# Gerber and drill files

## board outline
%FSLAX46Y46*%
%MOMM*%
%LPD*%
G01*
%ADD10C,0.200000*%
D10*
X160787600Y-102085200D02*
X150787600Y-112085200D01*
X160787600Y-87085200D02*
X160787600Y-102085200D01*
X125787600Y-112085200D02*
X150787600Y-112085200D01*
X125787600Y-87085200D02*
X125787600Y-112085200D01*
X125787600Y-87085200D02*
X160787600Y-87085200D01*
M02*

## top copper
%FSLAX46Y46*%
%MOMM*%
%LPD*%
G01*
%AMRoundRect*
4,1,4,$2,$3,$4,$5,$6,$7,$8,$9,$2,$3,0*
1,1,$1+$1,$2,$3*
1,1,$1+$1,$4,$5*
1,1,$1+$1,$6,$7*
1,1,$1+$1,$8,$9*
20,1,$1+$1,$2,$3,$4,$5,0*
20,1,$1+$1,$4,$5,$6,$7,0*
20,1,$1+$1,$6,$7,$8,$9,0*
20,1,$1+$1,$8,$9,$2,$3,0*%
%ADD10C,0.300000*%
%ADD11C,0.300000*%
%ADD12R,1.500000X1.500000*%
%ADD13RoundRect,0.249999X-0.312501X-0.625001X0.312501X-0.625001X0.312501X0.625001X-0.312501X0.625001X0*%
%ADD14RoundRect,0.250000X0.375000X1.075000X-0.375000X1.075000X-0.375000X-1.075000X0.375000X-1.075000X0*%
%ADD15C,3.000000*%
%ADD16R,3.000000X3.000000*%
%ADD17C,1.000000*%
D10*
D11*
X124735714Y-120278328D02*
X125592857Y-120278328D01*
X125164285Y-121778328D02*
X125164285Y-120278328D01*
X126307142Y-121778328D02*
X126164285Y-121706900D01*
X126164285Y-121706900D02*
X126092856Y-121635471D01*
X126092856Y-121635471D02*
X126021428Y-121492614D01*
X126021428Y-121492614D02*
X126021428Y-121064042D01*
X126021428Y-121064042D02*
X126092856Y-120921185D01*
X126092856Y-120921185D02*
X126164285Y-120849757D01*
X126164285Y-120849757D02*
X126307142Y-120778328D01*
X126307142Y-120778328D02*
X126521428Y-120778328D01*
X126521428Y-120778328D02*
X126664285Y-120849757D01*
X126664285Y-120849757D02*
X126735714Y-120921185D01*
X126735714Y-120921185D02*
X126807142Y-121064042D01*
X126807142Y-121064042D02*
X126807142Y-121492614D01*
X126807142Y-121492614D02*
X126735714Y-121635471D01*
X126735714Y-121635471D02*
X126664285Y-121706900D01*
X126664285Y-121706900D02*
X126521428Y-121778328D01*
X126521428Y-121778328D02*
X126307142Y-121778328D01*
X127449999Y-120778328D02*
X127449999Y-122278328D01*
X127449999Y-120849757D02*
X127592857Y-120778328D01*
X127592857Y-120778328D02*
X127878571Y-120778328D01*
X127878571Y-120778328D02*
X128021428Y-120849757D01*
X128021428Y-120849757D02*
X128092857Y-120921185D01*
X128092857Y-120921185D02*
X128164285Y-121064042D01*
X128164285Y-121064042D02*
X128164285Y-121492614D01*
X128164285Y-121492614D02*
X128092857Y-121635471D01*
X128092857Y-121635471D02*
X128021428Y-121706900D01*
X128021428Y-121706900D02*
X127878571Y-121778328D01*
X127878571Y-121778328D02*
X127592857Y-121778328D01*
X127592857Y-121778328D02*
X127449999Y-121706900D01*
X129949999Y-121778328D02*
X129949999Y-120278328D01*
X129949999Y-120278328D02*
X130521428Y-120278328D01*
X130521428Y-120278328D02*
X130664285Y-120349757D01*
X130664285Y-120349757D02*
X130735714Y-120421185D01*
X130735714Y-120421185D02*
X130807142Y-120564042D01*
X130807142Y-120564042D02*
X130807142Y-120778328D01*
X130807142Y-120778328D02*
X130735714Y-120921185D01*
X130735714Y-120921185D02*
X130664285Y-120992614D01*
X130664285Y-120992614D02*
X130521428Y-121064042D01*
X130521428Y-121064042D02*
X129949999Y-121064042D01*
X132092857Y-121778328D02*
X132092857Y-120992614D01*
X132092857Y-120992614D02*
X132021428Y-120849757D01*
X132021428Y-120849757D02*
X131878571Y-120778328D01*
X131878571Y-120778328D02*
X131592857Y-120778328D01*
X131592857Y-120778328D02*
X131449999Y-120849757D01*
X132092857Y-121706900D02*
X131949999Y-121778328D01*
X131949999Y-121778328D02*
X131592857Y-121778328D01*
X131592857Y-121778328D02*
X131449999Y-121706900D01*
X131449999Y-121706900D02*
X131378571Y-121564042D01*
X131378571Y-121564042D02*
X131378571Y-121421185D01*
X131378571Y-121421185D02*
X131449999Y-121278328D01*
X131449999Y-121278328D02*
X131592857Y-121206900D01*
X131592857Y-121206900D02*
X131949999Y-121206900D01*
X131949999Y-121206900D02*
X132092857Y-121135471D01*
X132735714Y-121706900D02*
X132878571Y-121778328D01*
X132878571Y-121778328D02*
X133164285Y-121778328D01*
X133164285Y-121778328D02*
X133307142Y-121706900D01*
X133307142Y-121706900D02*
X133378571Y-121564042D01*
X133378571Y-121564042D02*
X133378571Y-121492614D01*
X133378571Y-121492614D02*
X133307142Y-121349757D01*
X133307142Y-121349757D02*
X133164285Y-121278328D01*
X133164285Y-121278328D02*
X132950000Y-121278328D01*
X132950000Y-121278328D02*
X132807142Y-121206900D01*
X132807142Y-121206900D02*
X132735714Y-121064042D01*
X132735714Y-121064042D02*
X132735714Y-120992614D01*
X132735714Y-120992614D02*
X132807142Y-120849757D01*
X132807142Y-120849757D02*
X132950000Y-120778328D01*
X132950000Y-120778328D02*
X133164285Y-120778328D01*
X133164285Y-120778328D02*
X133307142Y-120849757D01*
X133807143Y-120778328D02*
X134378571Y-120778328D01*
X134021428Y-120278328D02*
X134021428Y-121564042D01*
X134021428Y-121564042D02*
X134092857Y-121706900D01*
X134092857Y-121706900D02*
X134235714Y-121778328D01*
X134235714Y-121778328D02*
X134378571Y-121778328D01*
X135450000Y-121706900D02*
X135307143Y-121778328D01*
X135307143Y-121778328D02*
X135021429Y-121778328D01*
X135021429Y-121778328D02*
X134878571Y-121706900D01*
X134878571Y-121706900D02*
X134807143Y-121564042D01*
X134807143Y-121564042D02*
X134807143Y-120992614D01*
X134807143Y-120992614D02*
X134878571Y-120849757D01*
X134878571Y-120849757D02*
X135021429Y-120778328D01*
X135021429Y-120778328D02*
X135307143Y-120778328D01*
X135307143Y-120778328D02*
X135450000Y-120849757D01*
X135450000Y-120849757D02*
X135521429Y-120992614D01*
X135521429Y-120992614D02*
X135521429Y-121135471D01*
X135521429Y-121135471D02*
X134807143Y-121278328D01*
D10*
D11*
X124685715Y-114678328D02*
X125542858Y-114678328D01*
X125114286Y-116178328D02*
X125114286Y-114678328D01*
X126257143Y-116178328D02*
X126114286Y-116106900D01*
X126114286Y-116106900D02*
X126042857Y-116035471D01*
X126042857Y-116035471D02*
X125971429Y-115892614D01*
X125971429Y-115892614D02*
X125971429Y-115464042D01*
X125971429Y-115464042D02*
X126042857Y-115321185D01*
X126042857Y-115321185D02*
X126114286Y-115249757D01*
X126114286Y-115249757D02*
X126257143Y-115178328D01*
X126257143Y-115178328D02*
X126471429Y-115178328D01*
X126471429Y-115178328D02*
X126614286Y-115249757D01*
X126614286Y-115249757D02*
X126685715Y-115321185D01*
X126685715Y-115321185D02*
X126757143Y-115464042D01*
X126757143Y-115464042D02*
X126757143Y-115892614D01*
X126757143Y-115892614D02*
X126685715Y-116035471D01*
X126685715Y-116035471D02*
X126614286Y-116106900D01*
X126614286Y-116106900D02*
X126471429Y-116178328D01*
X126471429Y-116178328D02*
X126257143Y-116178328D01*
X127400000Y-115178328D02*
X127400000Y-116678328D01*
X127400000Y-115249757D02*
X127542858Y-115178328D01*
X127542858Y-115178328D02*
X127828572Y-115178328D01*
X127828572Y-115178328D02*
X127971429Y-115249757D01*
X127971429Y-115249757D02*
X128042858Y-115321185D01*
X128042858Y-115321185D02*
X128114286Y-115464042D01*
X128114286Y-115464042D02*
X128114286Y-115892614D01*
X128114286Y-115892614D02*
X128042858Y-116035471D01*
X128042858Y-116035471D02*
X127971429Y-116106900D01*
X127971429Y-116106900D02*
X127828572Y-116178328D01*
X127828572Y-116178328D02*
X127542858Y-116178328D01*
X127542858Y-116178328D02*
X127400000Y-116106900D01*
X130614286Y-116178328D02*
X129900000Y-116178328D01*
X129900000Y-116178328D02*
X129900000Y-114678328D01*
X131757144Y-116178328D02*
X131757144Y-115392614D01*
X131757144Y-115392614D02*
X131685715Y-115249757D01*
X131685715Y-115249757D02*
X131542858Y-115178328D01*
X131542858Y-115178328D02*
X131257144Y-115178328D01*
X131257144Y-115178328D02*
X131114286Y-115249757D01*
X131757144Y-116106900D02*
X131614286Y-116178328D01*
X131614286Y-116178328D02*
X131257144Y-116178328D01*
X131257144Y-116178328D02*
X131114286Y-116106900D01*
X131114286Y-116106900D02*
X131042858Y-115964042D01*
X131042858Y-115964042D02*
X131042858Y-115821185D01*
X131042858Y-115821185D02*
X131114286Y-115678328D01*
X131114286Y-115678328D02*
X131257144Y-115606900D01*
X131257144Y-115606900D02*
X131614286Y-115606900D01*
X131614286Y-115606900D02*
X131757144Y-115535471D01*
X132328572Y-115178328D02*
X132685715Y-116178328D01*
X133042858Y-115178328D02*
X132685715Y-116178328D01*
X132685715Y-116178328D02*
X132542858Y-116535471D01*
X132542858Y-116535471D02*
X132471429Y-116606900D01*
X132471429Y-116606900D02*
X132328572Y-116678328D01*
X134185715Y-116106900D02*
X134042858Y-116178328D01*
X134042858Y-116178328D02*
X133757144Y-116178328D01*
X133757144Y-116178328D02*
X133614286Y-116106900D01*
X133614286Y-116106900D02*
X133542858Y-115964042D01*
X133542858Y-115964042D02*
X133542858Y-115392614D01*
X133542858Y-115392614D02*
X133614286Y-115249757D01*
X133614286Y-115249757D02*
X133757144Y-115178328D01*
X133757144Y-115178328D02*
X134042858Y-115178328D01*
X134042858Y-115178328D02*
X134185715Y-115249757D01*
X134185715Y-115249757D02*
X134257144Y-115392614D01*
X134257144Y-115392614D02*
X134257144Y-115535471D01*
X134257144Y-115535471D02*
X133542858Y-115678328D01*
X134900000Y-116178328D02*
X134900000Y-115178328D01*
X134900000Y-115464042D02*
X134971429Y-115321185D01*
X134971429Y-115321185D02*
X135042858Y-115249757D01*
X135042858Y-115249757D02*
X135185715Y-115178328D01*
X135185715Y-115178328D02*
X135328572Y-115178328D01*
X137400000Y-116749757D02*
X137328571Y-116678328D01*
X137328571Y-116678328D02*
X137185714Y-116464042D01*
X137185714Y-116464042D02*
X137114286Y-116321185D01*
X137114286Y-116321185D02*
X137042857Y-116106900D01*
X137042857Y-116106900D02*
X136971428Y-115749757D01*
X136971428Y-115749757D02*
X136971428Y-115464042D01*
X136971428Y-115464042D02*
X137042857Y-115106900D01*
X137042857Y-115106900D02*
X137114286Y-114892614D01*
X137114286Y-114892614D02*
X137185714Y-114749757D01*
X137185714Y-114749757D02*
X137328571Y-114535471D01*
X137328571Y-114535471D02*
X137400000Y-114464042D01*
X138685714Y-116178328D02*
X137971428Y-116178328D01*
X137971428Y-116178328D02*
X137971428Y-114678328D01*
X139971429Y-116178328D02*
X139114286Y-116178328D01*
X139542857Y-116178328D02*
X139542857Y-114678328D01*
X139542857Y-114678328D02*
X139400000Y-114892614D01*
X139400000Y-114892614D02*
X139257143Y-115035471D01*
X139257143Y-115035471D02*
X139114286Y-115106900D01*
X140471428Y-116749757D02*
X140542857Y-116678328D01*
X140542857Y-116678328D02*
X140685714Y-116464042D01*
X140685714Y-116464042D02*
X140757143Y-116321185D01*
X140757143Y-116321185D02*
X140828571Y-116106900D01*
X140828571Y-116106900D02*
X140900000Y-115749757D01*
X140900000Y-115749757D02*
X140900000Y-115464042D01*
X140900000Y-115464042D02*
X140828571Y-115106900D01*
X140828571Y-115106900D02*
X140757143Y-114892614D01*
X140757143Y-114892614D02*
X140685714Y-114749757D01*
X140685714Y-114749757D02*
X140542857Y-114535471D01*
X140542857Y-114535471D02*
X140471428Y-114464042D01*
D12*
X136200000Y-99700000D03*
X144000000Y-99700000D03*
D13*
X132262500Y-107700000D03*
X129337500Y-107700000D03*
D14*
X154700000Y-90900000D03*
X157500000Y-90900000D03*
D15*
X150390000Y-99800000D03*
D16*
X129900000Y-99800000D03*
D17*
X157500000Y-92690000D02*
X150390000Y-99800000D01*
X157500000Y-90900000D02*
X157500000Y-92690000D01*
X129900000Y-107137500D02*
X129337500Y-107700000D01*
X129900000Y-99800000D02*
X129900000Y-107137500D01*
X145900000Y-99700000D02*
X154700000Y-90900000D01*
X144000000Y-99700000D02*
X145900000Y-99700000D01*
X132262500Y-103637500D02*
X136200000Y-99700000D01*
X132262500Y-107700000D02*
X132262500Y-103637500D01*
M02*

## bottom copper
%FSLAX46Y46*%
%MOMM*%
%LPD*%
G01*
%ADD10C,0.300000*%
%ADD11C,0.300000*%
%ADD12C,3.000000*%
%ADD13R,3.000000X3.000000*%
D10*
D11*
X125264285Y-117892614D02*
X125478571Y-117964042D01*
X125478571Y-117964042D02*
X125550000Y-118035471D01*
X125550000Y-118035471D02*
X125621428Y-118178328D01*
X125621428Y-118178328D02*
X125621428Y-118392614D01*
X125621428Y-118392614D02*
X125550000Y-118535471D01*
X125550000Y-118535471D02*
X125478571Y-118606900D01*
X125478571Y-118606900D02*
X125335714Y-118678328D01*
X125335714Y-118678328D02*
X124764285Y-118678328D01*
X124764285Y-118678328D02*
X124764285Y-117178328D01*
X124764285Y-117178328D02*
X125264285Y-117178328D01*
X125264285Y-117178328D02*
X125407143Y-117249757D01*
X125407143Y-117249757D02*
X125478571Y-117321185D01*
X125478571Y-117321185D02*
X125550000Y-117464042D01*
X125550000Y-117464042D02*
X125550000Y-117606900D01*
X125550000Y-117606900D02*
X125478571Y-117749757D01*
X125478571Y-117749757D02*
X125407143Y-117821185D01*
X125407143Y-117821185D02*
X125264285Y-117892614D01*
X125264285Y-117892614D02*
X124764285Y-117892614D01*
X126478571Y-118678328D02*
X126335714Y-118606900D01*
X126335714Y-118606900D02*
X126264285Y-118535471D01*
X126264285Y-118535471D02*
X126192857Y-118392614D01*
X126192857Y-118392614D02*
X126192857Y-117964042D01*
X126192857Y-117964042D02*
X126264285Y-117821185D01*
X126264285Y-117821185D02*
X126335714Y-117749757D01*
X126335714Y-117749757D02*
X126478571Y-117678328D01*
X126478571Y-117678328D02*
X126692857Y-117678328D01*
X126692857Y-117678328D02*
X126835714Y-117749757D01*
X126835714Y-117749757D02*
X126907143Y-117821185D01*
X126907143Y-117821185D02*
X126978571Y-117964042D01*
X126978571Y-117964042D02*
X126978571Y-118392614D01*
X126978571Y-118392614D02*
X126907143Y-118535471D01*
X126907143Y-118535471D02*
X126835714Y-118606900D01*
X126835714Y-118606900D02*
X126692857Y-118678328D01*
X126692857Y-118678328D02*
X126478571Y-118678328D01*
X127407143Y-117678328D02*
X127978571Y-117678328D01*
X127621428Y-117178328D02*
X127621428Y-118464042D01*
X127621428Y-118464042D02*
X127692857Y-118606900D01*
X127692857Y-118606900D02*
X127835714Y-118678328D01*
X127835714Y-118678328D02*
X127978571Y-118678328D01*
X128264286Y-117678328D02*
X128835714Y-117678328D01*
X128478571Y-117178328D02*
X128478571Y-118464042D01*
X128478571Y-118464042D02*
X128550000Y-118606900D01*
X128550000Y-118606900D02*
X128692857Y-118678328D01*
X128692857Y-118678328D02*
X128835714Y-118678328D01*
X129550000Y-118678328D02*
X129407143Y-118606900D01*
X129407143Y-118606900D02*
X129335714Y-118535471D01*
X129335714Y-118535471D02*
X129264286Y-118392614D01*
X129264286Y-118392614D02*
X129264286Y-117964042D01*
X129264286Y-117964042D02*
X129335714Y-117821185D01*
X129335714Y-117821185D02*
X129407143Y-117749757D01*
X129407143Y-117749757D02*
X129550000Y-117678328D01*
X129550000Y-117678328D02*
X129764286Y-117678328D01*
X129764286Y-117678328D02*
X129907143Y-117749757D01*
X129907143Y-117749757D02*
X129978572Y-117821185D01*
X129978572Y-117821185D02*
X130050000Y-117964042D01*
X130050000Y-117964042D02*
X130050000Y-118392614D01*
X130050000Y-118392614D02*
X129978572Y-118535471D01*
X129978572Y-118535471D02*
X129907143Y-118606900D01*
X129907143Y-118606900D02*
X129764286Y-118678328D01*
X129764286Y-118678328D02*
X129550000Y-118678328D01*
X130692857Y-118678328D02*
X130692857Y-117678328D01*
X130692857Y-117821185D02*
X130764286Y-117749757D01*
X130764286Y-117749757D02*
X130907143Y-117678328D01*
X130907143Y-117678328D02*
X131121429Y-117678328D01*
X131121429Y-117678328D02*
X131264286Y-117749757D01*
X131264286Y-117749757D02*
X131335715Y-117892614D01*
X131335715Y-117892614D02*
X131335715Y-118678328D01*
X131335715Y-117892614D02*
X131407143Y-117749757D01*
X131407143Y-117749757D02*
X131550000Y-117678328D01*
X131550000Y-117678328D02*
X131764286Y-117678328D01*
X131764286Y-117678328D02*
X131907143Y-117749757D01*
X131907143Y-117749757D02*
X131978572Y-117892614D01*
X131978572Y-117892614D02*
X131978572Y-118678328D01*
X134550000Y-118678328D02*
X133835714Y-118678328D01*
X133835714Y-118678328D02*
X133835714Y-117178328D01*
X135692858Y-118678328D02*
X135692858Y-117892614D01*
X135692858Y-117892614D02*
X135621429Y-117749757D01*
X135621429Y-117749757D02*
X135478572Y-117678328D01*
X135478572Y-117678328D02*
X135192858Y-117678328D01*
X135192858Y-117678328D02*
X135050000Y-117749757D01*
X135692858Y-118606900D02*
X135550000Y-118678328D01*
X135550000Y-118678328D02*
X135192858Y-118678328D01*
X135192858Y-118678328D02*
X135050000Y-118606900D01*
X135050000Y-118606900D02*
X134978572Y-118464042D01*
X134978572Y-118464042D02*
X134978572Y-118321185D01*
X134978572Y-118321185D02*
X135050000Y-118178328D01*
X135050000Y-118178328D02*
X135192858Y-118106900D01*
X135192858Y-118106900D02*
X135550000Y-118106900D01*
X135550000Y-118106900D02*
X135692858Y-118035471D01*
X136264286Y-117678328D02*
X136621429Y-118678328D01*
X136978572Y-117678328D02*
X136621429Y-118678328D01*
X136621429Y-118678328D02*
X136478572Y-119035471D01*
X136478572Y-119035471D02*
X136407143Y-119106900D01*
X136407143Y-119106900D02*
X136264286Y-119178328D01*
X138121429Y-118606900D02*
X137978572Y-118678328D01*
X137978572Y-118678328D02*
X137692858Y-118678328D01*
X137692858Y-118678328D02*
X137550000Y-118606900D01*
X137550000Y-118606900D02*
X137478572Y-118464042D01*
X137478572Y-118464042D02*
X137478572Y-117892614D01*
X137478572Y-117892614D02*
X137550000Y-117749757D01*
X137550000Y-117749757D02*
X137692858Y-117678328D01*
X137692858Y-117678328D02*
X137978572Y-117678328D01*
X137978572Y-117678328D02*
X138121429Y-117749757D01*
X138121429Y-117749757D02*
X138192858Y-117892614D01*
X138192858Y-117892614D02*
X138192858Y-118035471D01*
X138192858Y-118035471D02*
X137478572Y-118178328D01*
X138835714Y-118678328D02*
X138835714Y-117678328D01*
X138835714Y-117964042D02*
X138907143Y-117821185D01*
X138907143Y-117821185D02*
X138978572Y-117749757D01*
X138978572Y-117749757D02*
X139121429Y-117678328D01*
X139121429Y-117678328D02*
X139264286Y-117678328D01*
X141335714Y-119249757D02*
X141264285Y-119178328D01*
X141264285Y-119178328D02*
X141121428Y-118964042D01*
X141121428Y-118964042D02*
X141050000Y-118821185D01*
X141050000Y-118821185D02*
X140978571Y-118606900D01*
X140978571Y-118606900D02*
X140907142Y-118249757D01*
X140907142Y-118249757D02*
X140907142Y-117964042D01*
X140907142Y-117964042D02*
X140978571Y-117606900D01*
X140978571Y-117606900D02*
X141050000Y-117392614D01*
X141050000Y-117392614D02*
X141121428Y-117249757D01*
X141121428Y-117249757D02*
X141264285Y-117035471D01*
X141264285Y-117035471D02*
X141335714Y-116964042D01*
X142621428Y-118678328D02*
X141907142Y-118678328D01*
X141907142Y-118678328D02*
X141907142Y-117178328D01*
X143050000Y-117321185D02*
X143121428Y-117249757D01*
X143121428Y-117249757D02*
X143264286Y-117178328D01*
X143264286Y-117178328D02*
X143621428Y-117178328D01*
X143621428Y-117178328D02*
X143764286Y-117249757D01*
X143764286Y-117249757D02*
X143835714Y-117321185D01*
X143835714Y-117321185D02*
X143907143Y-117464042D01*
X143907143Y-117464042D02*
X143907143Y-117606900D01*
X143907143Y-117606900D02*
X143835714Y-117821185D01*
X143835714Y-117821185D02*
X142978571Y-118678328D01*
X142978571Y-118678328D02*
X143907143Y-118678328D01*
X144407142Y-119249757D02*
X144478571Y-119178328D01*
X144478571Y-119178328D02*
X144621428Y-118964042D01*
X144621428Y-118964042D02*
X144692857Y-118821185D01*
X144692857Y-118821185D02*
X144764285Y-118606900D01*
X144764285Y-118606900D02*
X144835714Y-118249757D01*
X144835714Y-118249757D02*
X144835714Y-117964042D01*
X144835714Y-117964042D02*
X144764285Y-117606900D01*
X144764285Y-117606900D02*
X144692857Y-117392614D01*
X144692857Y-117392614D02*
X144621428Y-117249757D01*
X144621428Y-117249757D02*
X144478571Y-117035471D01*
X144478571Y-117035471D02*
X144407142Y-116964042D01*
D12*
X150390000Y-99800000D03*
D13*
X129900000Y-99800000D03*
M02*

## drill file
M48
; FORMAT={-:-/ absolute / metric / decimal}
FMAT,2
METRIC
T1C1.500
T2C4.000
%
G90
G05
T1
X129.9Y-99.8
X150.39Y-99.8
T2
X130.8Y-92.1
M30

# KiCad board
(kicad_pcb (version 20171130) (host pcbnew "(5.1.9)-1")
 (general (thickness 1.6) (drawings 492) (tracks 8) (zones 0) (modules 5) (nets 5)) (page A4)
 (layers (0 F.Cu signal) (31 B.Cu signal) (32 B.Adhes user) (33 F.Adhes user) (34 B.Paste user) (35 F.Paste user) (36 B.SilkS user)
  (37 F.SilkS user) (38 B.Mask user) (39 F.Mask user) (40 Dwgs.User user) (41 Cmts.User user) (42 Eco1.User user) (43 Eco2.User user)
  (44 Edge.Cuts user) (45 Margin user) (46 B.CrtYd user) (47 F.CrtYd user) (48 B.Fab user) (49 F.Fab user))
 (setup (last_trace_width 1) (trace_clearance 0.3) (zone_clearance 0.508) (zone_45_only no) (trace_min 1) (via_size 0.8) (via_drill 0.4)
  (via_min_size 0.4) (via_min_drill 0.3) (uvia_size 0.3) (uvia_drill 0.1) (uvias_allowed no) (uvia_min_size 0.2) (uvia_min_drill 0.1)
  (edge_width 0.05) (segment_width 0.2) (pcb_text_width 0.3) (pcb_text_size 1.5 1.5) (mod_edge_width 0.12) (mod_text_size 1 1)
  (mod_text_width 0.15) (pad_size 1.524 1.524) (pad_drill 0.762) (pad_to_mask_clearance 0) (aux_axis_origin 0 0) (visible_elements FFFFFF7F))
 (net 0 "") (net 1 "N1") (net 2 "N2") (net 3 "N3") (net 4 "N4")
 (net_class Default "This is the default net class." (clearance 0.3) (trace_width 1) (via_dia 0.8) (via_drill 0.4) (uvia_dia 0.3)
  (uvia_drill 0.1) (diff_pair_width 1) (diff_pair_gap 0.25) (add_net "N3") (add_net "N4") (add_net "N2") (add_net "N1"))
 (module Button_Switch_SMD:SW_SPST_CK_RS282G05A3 (layer F.Cu) (at 140.1 99.7 180)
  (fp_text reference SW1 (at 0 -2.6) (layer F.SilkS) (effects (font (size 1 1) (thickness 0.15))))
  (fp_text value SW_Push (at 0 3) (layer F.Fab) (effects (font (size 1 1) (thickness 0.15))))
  (pad 2 smd rect (at 3.9 0 180) (size 1.5 1.5) (layers F.Cu F.Paste F.Mask) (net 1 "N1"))
  (pad 1 smd rect (at -3.9 0 180) (size 1.5 1.5) (layers F.Cu F.Paste F.Mask) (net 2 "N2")))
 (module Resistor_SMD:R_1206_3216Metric (layer F.Cu) (at 130.8 107.7)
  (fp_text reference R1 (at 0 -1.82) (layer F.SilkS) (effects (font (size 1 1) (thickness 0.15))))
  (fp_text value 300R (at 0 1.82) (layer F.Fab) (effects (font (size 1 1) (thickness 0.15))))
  (pad 2 smd roundrect (at 1.4625 0) (size 1.125 1.75) (layers F.Cu F.Paste F.Mask) (roundrect_rratio 0.2222213333333333) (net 1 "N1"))
  (pad 1 smd roundrect (at -1.4625 0) (size 1.125 1.75) (layers F.Cu F.Paste F.Mask) (roundrect_rratio 0.2222213333333333) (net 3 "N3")))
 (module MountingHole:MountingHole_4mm (layer F.Cu) (at 130.8 92.1)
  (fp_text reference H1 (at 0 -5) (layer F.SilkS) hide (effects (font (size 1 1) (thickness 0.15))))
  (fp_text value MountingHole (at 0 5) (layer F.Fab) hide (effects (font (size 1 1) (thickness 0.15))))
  (pad 1 np_thru_hole circle (at 0 0) (size 4 4) (drill 4) (layers *.Cu *.Mask)))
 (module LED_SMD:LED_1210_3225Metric (layer F.Cu) (at 156.1 90.9 180)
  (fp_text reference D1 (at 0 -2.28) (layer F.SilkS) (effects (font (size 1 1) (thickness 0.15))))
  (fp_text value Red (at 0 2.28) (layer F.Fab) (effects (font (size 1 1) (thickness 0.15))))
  (pad 2 smd roundrect (at 1.4 0 180) (size 1.25 2.65) (layers F.Cu F.Paste F.Mask) (roundrect_rratio 0.2) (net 2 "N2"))
  (pad 1 smd roundrect (at -1.4 0 180) (size 1.25 2.65) (layers F.Cu F.Paste F.Mask) (roundrect_rratio 0.2) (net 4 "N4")))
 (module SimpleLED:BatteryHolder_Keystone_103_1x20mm (layer B.Cu) (at 129.9 99.8)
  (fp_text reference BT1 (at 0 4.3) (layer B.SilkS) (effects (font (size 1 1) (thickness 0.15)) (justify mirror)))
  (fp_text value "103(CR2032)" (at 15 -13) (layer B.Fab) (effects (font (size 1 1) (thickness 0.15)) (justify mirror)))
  (pad 2 thru_hole circle (at 20.49 0) (size 3 3) (drill 1.5) (layers *.Cu *.Mask) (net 4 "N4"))
  (pad 1 thru_hole rect (at 0 0) (size 3 3) (drill 1.5) (layers *.Cu *.Mask) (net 3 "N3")))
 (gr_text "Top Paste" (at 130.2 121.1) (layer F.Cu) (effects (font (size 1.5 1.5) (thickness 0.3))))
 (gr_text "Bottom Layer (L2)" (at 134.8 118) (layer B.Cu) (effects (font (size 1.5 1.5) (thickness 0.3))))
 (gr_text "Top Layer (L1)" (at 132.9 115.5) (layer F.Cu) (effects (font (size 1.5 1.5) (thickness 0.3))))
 (gr_line (start 160.7876 102.0852) (end 150.7876 112.0852) (layer Edge.Cuts) (width 0.2))
 (gr_line (start 160.7876 87.0852) (end 160.7876 102.0852) (layer Edge.Cuts) (width 0.2))
 (gr_line (start 125.7876 112.0852) (end 150.7876 112.0852) (layer Edge.Cuts) (width 0.2))
 (gr_line (start 125.7876 87.0852) (end 125.7876 112.0852) (layer Edge.Cuts) (width 0.2))
 (gr_line (start 125.7876 87.0852) (end 160.7876 87.0852) (layer Edge.Cuts) (width 0.2))
 (segment (start 157.5 92.69) (end 150.39 99.8) (width 1) (layer F.Cu) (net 4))
 (segment (start 157.5 90.9) (end 157.5 92.69) (width 1) (layer F.Cu) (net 4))
 (segment (start 129.9 107.1375) (end 129.3375 107.7) (width 1) (layer F.Cu) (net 3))
 (segment (start 129.9 99.8) (end 129.9 107.1375) (width 1) (layer F.Cu) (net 3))
 (segment (start 145.9 99.7) (end 154.7 90.9) (width 1) (layer F.Cu) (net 2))
 (segment (start 144 99.7) (end 145.9 99.7) (width 1) (layer F.Cu) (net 2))
 (segment (start 132.2625 103.6375) (end 136.2 99.7) (width 1) (layer F.Cu) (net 1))
 (segment (start 132.2625 107.7) (end 132.2625 103.6375) (width 1) (layer F.Cu) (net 1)))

